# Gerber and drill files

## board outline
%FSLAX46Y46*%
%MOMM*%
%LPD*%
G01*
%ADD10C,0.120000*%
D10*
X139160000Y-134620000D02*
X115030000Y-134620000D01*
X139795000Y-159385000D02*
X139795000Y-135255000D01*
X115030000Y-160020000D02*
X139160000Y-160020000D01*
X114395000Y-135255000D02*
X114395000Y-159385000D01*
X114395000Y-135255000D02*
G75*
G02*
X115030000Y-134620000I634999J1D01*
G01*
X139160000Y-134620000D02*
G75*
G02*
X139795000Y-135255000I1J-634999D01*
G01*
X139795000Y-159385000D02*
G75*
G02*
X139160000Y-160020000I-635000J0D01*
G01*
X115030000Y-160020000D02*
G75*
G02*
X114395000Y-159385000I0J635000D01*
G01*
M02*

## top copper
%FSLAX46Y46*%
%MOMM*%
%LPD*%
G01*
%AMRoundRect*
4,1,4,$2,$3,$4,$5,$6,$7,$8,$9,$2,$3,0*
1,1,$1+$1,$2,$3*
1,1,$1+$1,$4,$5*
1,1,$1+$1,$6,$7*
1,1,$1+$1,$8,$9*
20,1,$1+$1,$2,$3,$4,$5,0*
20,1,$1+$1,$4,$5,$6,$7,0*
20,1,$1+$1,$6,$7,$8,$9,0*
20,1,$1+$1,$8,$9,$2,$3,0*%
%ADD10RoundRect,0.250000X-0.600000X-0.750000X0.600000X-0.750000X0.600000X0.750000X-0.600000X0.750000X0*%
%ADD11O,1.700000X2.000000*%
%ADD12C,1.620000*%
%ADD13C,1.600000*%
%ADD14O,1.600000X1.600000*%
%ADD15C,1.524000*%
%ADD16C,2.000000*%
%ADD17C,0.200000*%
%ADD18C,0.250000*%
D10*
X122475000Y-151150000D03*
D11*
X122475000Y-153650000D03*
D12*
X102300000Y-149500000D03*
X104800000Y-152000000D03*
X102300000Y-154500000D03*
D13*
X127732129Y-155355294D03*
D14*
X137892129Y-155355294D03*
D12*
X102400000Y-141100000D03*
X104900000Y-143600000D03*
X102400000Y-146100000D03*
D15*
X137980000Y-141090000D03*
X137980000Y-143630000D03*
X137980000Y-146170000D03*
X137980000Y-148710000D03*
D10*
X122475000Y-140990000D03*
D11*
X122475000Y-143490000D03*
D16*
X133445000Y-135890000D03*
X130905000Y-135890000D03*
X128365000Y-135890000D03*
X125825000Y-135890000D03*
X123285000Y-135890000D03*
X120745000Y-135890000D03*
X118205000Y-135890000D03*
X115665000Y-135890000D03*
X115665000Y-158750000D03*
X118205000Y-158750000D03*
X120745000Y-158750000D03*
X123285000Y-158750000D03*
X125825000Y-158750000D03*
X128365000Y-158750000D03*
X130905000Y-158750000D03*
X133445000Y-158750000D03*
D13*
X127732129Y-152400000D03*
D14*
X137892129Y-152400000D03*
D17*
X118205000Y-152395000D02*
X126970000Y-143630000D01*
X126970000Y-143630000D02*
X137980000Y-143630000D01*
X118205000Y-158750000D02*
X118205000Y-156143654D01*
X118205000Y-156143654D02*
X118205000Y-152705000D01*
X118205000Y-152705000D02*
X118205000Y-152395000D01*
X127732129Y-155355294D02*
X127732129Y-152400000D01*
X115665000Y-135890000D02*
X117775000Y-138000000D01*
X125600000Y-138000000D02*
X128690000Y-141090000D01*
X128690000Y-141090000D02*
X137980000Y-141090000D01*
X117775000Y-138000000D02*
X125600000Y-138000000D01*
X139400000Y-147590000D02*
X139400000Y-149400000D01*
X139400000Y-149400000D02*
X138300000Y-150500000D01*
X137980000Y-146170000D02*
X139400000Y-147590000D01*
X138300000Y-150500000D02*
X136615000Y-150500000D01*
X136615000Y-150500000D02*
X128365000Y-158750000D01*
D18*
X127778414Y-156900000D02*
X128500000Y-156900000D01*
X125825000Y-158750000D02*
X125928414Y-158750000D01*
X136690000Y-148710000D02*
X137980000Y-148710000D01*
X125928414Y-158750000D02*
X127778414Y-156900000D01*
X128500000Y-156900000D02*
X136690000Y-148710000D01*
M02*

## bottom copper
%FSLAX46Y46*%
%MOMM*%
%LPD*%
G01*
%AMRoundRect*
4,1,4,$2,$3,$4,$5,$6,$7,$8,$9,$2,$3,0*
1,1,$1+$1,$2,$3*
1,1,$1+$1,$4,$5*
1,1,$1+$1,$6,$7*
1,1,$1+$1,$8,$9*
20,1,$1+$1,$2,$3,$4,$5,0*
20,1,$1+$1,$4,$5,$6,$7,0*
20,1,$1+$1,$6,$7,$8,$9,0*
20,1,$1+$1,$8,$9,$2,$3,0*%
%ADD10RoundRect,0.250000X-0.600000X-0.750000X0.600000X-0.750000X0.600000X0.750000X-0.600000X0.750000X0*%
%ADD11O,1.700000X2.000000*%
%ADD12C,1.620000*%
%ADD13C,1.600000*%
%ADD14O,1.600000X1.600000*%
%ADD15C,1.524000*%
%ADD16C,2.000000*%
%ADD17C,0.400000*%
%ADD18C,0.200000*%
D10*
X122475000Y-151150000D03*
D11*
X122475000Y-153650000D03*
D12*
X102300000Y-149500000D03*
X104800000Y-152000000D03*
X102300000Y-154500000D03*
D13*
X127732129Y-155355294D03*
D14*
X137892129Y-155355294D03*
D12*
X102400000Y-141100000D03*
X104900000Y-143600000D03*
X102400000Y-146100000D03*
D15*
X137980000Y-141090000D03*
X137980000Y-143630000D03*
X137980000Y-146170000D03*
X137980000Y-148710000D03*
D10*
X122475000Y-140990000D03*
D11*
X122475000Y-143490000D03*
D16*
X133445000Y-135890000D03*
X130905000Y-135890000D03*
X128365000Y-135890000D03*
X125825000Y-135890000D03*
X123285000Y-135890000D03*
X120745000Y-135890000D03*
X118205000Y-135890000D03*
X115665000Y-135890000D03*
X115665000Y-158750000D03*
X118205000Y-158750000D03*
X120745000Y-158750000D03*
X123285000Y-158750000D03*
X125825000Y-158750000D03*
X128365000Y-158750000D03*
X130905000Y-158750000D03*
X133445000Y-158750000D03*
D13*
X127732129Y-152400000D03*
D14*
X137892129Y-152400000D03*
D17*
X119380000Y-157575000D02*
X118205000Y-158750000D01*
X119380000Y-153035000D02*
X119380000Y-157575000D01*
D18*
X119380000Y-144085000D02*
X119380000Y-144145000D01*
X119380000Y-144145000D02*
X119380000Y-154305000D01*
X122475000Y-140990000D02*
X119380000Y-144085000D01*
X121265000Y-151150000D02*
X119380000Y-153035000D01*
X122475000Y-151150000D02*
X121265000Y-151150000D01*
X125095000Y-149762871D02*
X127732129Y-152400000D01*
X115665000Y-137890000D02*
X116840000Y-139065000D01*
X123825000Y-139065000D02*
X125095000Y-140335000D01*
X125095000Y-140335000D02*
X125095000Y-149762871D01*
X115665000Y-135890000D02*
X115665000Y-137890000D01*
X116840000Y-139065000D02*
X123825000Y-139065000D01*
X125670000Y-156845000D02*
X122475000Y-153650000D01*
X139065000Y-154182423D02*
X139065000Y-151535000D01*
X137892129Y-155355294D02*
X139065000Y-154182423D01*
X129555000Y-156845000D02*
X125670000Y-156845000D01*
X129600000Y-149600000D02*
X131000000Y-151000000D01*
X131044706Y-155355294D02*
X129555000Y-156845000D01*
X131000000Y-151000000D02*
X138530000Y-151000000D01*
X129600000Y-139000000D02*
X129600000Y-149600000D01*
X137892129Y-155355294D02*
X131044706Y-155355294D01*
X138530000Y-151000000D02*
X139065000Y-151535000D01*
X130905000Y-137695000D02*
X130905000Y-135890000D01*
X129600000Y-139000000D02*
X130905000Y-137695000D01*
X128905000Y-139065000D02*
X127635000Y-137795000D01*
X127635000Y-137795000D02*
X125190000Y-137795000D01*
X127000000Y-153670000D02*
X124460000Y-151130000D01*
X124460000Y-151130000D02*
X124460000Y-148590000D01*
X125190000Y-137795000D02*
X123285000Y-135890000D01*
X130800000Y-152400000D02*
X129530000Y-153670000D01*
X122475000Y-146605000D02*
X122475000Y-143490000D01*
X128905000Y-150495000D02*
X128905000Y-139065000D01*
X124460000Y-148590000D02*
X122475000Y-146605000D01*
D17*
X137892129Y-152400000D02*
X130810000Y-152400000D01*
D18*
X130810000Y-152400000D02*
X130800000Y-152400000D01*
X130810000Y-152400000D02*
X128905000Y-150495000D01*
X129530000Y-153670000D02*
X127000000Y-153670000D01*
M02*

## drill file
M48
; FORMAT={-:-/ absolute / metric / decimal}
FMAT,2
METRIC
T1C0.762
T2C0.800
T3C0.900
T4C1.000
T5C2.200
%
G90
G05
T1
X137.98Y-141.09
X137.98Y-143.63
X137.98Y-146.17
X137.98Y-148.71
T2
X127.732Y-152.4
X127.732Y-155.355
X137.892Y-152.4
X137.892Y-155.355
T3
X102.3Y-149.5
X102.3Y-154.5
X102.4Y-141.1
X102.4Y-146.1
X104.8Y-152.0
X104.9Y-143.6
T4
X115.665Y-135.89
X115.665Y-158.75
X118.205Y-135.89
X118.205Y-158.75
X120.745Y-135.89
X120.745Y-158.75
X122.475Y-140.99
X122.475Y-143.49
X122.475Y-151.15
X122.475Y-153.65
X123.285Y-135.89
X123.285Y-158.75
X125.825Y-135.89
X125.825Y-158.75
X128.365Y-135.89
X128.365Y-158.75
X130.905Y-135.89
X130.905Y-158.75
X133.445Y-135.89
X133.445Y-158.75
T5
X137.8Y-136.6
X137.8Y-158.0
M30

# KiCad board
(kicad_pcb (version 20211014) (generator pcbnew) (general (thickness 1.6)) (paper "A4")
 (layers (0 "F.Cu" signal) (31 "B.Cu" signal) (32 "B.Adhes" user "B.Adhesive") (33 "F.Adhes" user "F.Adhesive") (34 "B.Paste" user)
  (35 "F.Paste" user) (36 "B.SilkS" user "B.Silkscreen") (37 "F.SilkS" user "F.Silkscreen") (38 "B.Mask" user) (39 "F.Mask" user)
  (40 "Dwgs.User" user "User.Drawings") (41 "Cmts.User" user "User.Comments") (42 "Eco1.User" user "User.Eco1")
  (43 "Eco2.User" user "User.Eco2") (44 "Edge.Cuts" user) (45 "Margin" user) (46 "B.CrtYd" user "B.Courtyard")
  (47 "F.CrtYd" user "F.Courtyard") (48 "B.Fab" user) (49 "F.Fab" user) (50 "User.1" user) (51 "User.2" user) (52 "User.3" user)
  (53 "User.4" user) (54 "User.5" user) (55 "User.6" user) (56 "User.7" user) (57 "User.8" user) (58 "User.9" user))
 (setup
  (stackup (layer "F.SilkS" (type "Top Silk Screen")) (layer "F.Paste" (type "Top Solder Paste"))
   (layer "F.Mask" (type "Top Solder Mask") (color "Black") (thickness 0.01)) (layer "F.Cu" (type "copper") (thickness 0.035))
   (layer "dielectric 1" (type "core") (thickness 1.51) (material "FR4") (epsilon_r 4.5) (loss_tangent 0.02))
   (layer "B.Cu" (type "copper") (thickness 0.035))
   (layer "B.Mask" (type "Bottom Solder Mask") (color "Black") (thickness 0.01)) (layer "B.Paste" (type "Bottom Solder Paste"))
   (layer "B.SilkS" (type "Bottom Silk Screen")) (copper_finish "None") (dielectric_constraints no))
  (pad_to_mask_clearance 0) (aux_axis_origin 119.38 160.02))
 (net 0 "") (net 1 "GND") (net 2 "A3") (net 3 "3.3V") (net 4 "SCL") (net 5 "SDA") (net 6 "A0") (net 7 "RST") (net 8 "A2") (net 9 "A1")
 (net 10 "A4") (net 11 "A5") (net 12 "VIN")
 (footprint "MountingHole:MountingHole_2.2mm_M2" (layer "F.Cu") (at 137.8 136.6)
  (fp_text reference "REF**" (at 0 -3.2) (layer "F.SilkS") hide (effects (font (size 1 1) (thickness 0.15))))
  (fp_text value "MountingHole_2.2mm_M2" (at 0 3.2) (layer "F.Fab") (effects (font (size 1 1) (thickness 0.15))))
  (pad "" np_thru_hole circle (at 0 0) (size 2.2 2.2) (drill 2.2) (layers *.Cu *.Mask)))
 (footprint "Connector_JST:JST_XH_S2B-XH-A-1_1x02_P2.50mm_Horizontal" (layer "F.Cu") (at 114.375 152.4 -90)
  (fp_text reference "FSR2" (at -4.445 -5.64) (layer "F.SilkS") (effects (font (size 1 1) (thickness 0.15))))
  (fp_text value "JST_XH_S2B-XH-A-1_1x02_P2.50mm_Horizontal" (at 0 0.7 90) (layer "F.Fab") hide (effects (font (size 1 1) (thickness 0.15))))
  (pad "1" thru_hole roundrect (at -1.25 -8.1) (size 1.7 2) (drill 1) (layers *.Cu *.Mask) (roundrect_rratio 0.1470588235) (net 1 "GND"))
  (pad "2" thru_hole oval (at 1.25 -8.1) (size 1.7 2) (drill 1) (layers *.Cu *.Mask) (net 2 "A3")))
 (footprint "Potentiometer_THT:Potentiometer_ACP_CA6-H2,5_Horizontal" (layer "F.Cu") (at 102.3 149.5)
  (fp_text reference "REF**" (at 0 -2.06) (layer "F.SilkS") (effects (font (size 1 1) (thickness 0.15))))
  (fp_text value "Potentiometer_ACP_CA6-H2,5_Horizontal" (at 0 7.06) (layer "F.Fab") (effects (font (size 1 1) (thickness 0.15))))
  (pad "1" thru_hole circle (at 0 0) (size 1.62 1.62) (drill 0.9) (layers F&B.Cu *.Mask))
  (pad "2" thru_hole circle (at 2.5 2.5) (size 1.62 1.62) (drill 0.9) (layers F&B.Cu *.Mask))
  (pad "3" thru_hole circle (at 0 5) (size 1.62 1.62) (drill 0.9) (layers F&B.Cu *.Mask)))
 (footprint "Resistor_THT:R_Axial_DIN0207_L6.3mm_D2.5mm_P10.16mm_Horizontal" (layer "F.Cu") (at 127.732129 155.355294)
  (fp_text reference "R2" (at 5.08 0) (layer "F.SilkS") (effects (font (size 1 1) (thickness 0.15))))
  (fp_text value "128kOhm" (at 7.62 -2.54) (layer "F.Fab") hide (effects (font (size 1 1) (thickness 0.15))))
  (pad "1" thru_hole circle (at 0 0) (size 1.6 1.6) (drill 0.8) (layers *.Cu *.Mask) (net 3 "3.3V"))
  (pad "2" thru_hole oval (at 10.16 0) (size 1.6 1.6) (drill 0.8) (layers *.Cu *.Mask) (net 2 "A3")))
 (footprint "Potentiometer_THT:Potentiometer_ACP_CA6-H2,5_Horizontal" (layer "F.Cu") (at 102.4 141.1)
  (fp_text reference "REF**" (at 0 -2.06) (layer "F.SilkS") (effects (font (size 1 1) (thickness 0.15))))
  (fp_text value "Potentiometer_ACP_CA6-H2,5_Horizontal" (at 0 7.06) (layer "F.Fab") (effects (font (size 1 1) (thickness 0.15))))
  (pad "1" thru_hole circle (at 0 0) (size 1.62 1.62) (drill 0.9) (layers *.Cu *.Mask))
  (pad "2" thru_hole circle (at 2.5 2.5) (size 1.62 1.62) (drill 0.9) (layers *.Cu *.Mask))
  (pad "3" thru_hole circle (at 0 5) (size 1.62 1.62) (drill 0.9) (layers *.Cu *.Mask)))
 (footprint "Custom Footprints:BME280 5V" (layer "F.Cu") (at 136.71 144.9 -90)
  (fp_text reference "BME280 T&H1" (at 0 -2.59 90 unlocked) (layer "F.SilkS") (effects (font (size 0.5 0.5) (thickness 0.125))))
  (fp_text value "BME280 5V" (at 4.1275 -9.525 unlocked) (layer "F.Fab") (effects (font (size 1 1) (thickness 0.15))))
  (pad "1" thru_hole circle (at -3.81 -1.27 180) (size 1.524 1.524) (drill 0.762) (layers *.Cu *.Mask) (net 3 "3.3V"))
  (pad "2" thru_hole circle (at -1.27 -1.27 180) (size 1.524 1.524) (drill 0.762) (layers *.Cu *.Mask) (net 1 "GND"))
  (pad "3" thru_hole circle (at 1.27 -1.27 180) (size 1.524 1.524) (drill 0.762) (layers *.Cu *.Mask) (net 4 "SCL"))
  (pad "4" thru_hole circle (at 3.81 -1.27 180) (size 1.524 1.524) (drill 0.762) (layers *.Cu *.Mask) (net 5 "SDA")))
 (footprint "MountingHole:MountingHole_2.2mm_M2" (layer "F.Cu") (at 137.8 158)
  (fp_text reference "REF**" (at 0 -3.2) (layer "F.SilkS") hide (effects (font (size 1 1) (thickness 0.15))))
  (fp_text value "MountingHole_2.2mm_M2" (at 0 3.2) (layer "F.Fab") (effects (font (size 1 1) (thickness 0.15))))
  (pad "" np_thru_hole circle (at 0 0) (size 2.2 2.2) (drill 2.2) (layers *.Cu *.Mask)))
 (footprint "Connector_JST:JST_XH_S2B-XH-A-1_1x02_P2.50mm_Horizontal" (layer "F.Cu") (at 114.375 142.24 -90)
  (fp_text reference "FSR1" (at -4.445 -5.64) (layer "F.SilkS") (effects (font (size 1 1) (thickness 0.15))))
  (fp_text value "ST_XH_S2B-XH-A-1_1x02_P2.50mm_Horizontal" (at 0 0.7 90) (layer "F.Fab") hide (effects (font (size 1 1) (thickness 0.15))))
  (pad "1" thru_hole roundrect (at -1.25 -8.1) (size 1.7 2) (drill 1) (layers *.Cu *.Mask) (roundrect_rratio 0.1470588235) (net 1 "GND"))
  (pad "2" thru_hole oval (at 1.25 -8.1) (size 1.7 2) (drill 1) (layers *.Cu *.Mask) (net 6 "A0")))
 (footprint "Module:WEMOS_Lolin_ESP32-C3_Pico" (layer "F.Cu") (at 114.395 147.32 -90)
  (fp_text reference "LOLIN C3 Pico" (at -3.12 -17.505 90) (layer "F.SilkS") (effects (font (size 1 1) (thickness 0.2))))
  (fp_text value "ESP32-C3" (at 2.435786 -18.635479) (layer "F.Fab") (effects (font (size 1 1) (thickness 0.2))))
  (fp_line (start -12.7 -24.765) (end -12.7 -0.635) (layer "Edge.Cuts") (width 0.12))
  (fp_line (start 12.065 -25.4) (end -12.065 -25.4) (layer "Edge.Cuts") (width 0.12))
  (fp_line (start 12.7 -0.635) (end 12.7 -24.765) (layer "Edge.Cuts") (width 0.12))
  (fp_line (start -12.065 0) (end 12.065 0) (layer "Edge.Cuts") (width 0.12))
  (fp_arc (start -12.065 0) (mid -12.514013 -0.185987) (end -12.7 -0.635) (layer "Edge.Cuts") (width 0.12))
  (fp_arc (start -12.7 -24.765) (mid -12.514013 -25.214013) (end -12.065 -25.4) (layer "Edge.Cuts") (width 0.12))
  (fp_arc (start 12.065 -25.4) (mid 12.514013 -25.214013) (end 12.7 -24.765) (layer "Edge.Cuts") (width 0.12))
  (fp_arc (start 12.7 -0.635) (mid 12.514013 -0.185987) (end 12.065 0) (layer "Edge.Cuts") (width 0.12))
  (pad "1" thru_hole circle (at -11.43 -19.05 270) (size 2 2) (drill 1) (layers *.Cu *.Mask) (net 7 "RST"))
  (pad "2" thru_hole circle (at -11.43 -16.51 270) (size 2 2) (drill 1) (layers *.Cu *.Mask) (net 2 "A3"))
  (pad "3" thru_hole circle (at -11.43 -13.97 270) (size 2 2) (drill 1) (layers *.Cu *.Mask) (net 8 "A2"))
  (pad "4" thru_hole circle (at -11.43 -11.43 270) (size 2 2) (drill 1) (layers *.Cu *.Mask) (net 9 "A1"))
  (pad "5" thru_hole circle (at -11.43 -8.89 270) (size 2 2) (drill 1) (layers *.Cu *.Mask) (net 6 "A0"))
  (pad "6" thru_hole circle (at -11.43 -6.35 270) (size 2 2) (drill 1) (layers *.Cu *.Mask) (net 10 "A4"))
  (pad "7" thru_hole circle (at -11.43 -3.81 270) (size 2 2) (drill 1) (layers *.Cu *.Mask) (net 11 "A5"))
  (pad "8" thru_hole circle (at -11.43 -1.27 270) (size 2 2) (drill 1) (layers *.Cu *.Mask) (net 3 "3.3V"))
  (pad "9" thru_hole circle (at 11.43 -1.27 270) (size 2 2) (drill 1) (layers *.Cu *.Mask) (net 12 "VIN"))
  (pad "10" thru_hole circle (at 11.43 -3.81 270) (size 2 2) (drill 1) (layers *.Cu *.Mask) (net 1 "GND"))
  (pad "11" thru_hole circle (at 11.43 -6.35 270) (size 2 2) (drill 1) (layers *.Cu *.Mask))
  (pad "12" thru_hole circle (at 11.43 -8.89 270) (size 2 2) (drill 1) (layers *.Cu *.Mask))
  (pad "13" thru_hole circle (at 11.43 -11.43 270) (size 2 2) (drill 1) (layers *.Cu *.Mask) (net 5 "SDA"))
  (pad "14" thru_hole circle (at 11.43 -13.97 270) (size 2 2) (drill 1) (layers *.Cu *.Mask) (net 4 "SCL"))
  (pad "15" thru_hole circle (at 11.43 -16.51 270) (size 2 2) (drill 1) (layers *.Cu *.Mask))
  (pad "16" thru_hole circle (at 11.43 -19.05 270) (size 2 2) (drill 1) (layers *.Cu *.Mask)))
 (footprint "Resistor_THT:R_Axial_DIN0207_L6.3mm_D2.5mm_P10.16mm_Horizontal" (layer "F.Cu") (at 127.732129 152.4)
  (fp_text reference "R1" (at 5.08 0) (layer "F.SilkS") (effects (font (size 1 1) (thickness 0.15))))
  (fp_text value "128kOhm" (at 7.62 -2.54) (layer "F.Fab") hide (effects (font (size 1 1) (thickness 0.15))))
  (pad "1" thru_hole circle (at 0 0) (size 1.6 1.6) (drill 0.8) (layers *.Cu *.Mask) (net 3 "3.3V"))
  (pad "2" thru_hole oval (at 10.16 0) (size 1.6 1.6) (drill 0.8) (layers *.Cu *.Mask) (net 6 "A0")))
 (segment (start 118.205 152.395) (end 126.97 143.63) (width 0.2) (layer "F.Cu") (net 1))
 (segment (start 126.97 143.63) (end 137.98 143.63) (width 0.2) (layer "F.Cu") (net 1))
 (segment (start 118.205 158.75) (end 118.205 156.143654) (width 0.2) (layer "F.Cu") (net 1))
 (segment (start 118.205 156.143654) (end 118.205 152.705) (width 0.2) (layer "F.Cu") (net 1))
 (segment (start 118.205 152.705) (end 118.205 152.395) (width 0.2) (layer "F.Cu") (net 1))
 (segment (start 119.38 157.575) (end 118.205 158.75) (width 0.4) (layer "B.Cu") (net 1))
 (segment (start 119.38 153.035) (end 119.38 157.575) (width 0.4) (layer "B.Cu") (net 1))
 (segment (start 119.38 144.085) (end 119.38 144.145) (width 0.2) (layer "B.Cu") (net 1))
 (segment (start 119.38 144.145) (end 119.38 154.305) (width 0.2) (layer "B.Cu") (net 1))
 (segment (start 122.475 140.99) (end 119.38 144.085) (width 0.2) (layer "B.Cu") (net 1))
 (segment (start 121.265 151.15) (end 119.38 153.035) (width 0.2) (layer "B.Cu") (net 1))
 (segment (start 122.475 151.15) (end 121.265 151.15) (width 0.2) (layer "B.Cu") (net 1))
 (segment (start 127.732129 155.355294) (end 127.732129 152.4) (width 0.2) (layer "F.Cu") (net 3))
 (segment (start 115.665 135.89) (end 117.775 138) (width 0.2) (layer "F.Cu") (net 3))
 (segment (start 125.6 138) (end 128.69 141.09) (width 0.2) (layer "F.Cu") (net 3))
 (segment (start 128.69 141.09) (end 137.98 141.09) (width 0.2) (layer "F.Cu") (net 3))
 (segment (start 117.775 138) (end 125.6 138) (width 0.2) (layer "F.Cu") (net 3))
 (segment (start 125.095 149.762871) (end 127.732129 152.4) (width 0.2) (layer "B.Cu") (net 3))
 (segment (start 115.665 137.89) (end 116.84 139.065) (width 0.2) (layer "B.Cu") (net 3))
 (segment (start 123.825 139.065) (end 125.095 140.335) (width 0.2) (layer "B.Cu") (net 3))
 (segment (start 125.095 140.335) (end 125.095 149.762871) (width 0.2) (layer "B.Cu") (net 3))
 (segment (start 115.665 135.89) (end 115.665 137.89) (width 0.2) (layer "B.Cu") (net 3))
 (segment (start 116.84 139.065) (end 123.825 139.065) (width 0.2) (layer "B.Cu") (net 3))
 (segment (start 125.67 156.845) (end 122.475 153.65) (width 0.2) (layer "B.Cu") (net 2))
 (segment (start 139.065 154.182423) (end 139.065 151.535) (width 0.2) (layer "B.Cu") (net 2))
 (segment (start 137.892129 155.355294) (end 139.065 154.182423) (width 0.2) (layer "B.Cu") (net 2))
 (segment (start 129.555 156.845) (end 125.67 156.845) (width 0.2) (layer "B.Cu") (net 2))
 (segment (start 129.6 149.6) (end 131 151) (width 0.2) (layer "B.Cu") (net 2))
 (segment (start 131.044706 155.355294) (end 129.555 156.845) (width 0.2) (layer "B.Cu") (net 2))
 (segment (start 131 151) (end 138.53 151) (width 0.2) (layer "B.Cu") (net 2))
 (segment (start 129.6 139) (end 129.6 149.6) (width 0.2) (layer "B.Cu") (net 2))
 (segment (start 137.892129 155.355294) (end 131.044706 155.355294) (width 0.2) (layer "B.Cu") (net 2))
 (segment (start 138.53 151) (end 139.065 151.535) (width 0.2) (layer "B.Cu") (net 2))
 (segment (start 130.905 137.695) (end 130.905 135.89) (width 0.2) (layer "B.Cu") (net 2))
 (segment (start 129.6 139) (end 130.905 137.695) (width 0.2) (layer "B.Cu") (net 2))
 (segment (start 128.905 139.065) (end 127.635 137.795) (width 0.2) (layer "B.Cu") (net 6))
 (segment (start 127.635 137.795) (end 125.19 137.795) (width 0.2) (layer "B.Cu") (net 6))
 (segment (start 127 153.67) (end 124.46 151.13) (width 0.2) (layer "B.Cu") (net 6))
 (segment (start 124.46 151.13) (end 124.46 148.59) (width 0.2) (layer "B.Cu") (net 6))
 (segment (start 125.19 137.795) (end 123.285 135.89) (width 0.2) (layer "B.Cu") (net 6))
 (segment (start 130.8 152.4) (end 129.53 153.67) (width 0.2) (layer "B.Cu") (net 6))
 (segment (start 122.475 146.605) (end 122.475 143.49) (width 0.2) (layer "B.Cu") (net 6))
 (segment (start 128.905 150.495) (end 128.905 139.065) (width 0.2) (layer "B.Cu") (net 6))
 (segment (start 124.46 148.59) (end 122.475 146.605) (width 0.2) (layer "B.Cu") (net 6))
 (segment (start 137.892129 152.4) (end 130.81 152.4) (width 0.4) (layer "B.Cu") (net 6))
 (segment (start 130.81 152.4) (end 130.8 152.4) (width 0.2) (layer "B.Cu") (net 6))
 (segment (start 130.81 152.4) (end 128.905 150.495) (width 0.2) (layer "B.Cu") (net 6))
 (segment (start 129.53 153.67) (end 127 153.67) (width 0.2) (layer "B.Cu") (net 6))
 (segment (start 139.4 147.59) (end 139.4 149.4) (width 0.2) (layer "F.Cu") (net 4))
 (segment (start 139.4 149.4) (end 138.3 150.5) (width 0.2) (layer "F.Cu") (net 4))
 (segment (start 137.98 146.17) (end 139.4 147.59) (width 0.2) (layer "F.Cu") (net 4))
 (segment (start 138.3 150.5) (end 136.615 150.5) (width 0.2) (layer "F.Cu") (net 4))
 (segment (start 136.615 150.5) (end 128.365 158.75) (width 0.2) (layer "F.Cu") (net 4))
 (segment (start 127.778414 156.9) (end 128.5 156.9) (width 0.25) (layer "F.Cu") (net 5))
 (segment (start 125.825 158.75) (end 125.928414 158.75) (width 0.25) (layer "F.Cu") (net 5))
 (segment (start 136.69 148.71) (end 137.98 148.71) (width 0.25) (layer "F.Cu") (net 5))
 (segment (start 125.928414 158.75) (end 127.778414 156.9) (width 0.25) (layer "F.Cu") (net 5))
 (segment (start 128.5 156.9) (end 136.69 148.71) (width 0.25) (layer "F.Cu") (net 5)))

